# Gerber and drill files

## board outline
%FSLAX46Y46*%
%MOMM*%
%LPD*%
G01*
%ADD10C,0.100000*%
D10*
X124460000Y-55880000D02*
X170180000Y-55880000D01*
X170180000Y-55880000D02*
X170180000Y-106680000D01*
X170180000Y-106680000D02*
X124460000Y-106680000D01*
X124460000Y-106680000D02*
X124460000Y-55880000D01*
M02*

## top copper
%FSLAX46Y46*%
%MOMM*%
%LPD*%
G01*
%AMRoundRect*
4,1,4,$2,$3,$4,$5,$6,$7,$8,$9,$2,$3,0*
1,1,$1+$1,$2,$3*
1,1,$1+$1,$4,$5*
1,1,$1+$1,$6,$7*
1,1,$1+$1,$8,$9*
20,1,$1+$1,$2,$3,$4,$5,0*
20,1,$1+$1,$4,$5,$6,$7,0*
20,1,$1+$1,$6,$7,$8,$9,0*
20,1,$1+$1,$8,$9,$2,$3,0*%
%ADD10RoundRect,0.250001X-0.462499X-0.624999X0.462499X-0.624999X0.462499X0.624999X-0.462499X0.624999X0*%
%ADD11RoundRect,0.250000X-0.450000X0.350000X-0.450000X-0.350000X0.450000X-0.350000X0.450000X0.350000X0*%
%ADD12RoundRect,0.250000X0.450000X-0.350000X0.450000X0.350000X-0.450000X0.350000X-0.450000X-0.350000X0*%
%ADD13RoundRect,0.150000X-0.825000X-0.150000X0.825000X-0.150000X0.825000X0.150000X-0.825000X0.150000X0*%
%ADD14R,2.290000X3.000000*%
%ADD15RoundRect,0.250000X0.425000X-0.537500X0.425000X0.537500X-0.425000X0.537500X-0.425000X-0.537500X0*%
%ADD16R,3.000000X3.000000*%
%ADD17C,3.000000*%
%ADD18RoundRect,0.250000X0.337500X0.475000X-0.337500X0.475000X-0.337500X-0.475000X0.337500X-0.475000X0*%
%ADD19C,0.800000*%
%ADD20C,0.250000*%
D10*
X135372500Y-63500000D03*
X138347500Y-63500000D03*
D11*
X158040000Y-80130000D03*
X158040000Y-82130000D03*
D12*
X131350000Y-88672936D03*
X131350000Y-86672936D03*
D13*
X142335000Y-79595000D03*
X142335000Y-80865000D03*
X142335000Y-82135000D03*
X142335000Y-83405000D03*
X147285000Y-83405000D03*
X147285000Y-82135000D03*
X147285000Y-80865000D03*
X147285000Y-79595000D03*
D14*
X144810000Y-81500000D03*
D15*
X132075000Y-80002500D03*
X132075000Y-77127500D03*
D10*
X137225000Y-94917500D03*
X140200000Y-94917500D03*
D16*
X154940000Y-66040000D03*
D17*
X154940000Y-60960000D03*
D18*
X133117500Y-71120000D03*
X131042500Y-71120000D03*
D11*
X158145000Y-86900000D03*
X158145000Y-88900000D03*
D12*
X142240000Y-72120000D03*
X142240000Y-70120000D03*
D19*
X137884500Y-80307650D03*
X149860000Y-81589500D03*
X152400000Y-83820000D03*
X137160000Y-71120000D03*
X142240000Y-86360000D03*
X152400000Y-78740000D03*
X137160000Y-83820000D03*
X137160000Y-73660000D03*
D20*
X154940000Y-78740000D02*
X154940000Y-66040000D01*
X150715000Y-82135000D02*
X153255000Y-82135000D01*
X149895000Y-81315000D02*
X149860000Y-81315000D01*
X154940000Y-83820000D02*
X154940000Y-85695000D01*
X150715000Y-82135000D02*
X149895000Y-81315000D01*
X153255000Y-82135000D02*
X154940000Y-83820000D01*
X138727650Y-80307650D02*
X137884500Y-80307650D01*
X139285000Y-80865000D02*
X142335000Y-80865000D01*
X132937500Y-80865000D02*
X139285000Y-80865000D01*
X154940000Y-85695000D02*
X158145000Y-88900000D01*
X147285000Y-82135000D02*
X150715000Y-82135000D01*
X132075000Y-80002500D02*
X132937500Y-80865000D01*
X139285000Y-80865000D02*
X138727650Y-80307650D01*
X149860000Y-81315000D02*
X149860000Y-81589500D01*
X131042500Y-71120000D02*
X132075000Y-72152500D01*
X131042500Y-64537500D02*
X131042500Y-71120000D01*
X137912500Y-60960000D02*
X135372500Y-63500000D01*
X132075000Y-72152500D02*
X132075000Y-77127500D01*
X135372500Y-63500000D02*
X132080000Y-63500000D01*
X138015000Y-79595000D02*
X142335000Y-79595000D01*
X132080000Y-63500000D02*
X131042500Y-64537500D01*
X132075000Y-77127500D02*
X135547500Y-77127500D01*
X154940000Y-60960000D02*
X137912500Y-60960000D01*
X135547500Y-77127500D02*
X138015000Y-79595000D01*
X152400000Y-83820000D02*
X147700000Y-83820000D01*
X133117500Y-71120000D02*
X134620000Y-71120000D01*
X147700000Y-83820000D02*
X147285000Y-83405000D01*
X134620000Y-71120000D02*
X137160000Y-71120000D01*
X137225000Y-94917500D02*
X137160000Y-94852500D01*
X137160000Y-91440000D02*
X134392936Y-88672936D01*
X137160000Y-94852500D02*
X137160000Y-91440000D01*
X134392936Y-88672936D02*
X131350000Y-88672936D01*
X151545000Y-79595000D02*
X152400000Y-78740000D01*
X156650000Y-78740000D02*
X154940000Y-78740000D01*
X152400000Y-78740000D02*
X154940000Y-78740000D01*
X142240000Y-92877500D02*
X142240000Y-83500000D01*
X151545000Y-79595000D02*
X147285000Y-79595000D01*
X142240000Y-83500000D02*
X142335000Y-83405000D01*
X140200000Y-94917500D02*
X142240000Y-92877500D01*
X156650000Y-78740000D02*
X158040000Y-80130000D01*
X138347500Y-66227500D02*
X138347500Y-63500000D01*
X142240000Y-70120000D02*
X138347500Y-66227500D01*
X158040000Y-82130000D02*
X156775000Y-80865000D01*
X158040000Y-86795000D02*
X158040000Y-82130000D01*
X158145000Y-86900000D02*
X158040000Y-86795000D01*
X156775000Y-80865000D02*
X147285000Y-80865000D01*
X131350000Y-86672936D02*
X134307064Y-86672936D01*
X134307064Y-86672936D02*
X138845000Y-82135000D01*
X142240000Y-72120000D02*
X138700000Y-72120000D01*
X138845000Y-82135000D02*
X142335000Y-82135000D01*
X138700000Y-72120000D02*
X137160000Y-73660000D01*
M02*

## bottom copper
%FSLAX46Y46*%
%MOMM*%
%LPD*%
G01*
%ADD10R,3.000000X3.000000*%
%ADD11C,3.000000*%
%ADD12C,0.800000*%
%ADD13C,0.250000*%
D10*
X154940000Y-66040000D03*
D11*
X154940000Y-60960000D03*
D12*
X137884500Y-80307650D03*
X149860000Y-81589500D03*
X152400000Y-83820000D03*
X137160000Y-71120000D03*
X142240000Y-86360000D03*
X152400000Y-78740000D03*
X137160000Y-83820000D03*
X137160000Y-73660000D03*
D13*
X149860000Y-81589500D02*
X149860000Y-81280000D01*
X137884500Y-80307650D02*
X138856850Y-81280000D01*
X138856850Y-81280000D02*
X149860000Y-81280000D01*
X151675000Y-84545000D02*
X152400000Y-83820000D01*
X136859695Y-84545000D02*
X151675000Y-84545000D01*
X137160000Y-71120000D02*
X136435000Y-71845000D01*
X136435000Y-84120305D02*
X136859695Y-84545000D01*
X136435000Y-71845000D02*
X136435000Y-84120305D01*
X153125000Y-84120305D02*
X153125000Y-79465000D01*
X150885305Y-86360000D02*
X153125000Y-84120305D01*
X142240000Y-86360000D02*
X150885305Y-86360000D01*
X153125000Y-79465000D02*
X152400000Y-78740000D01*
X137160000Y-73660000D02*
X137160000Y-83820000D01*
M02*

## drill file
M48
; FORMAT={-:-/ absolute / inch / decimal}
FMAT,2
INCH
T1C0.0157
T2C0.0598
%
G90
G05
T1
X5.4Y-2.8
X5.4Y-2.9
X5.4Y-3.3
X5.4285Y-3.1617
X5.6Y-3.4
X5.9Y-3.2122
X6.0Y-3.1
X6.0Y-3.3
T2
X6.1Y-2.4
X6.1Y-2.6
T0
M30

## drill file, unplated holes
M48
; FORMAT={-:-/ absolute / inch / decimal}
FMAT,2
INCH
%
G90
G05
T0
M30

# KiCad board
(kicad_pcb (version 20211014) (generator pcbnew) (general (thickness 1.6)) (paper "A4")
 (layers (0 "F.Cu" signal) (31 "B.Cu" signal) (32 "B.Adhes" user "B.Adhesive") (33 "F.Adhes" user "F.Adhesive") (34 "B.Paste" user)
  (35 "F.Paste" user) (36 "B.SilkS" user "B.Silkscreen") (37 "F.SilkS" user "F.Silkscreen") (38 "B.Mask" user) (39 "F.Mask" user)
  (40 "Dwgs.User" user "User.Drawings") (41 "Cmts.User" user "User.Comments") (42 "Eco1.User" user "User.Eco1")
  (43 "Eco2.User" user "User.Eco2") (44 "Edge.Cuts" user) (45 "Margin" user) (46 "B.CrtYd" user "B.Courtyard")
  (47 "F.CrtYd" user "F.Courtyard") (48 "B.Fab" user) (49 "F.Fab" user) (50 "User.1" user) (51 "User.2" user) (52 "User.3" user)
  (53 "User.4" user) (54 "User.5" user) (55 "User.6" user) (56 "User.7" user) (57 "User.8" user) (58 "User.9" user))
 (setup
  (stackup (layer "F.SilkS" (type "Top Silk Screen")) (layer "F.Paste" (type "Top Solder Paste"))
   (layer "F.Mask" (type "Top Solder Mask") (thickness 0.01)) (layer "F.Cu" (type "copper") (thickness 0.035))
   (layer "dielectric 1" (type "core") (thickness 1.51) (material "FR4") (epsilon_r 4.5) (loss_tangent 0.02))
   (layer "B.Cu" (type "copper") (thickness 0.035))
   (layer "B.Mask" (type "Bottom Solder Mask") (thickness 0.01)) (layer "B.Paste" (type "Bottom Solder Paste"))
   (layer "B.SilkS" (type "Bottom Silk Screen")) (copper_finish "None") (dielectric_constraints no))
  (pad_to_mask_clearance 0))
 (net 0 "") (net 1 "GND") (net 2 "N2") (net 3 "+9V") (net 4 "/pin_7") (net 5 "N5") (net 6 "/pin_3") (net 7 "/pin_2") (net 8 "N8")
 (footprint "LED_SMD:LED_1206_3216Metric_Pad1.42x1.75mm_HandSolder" (layer "F.Cu") (at 136.86 63.5)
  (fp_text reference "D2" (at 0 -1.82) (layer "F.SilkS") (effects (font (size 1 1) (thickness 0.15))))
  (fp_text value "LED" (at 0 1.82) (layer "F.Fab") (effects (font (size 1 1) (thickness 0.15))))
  (pad "1" smd roundrect (at -1.4875 0) (size 1.425 1.75) (layers "F.Cu" "F.Paste" "F.Mask") (roundrect_rratio 0.175439) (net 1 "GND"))
  (pad "2" smd roundrect (at 1.4875 0) (size 1.425 1.75) (layers "F.Cu" "F.Paste" "F.Mask") (roundrect_rratio 0.175439) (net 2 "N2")))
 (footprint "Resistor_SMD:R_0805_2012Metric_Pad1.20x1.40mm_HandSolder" (layer "F.Cu") (at 158.04 81.13 -90)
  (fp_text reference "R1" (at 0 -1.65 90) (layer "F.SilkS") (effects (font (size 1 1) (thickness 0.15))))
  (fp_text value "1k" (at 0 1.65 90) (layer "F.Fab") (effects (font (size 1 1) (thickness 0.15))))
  (pad "1" smd roundrect (at -1 0 270) (size 1.2 1.4) (layers "F.Cu" "F.Paste" "F.Mask") (roundrect_rratio 0.208333) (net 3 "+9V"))
  (pad "2" smd roundrect (at 1 0 270) (size 1.2 1.4) (layers "F.Cu" "F.Paste" "F.Mask") (roundrect_rratio 0.208333) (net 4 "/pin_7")))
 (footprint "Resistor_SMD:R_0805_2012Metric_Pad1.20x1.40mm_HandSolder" (layer "F.Cu") (at 131.35 87.672936 90)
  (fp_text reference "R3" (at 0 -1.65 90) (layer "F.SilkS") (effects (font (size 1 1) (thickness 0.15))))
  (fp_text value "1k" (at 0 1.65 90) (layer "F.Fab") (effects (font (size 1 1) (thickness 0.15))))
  (pad "1" smd roundrect (at -1 0 90) (size 1.2 1.4) (layers "F.Cu" "F.Paste" "F.Mask") (roundrect_rratio 0.208333) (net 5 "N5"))
  (pad "2" smd roundrect (at 1 0 90) (size 1.2 1.4) (layers "F.Cu" "F.Paste" "F.Mask") (roundrect_rratio 0.208333) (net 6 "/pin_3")))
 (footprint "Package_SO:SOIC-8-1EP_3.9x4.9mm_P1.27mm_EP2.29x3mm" (layer "F.Cu") (at 144.81 81.5)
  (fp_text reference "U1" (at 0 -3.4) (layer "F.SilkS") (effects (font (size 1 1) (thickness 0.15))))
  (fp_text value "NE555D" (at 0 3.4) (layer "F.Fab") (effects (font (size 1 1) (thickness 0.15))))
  (pad "" smd roundrect (at -0.57 -0.75) (size 0.92 1.21) (layers "F.Paste") (roundrect_rratio 0.25))
  (pad "" smd roundrect (at 0.57 0.75) (size 0.92 1.21) (layers "F.Paste") (roundrect_rratio 0.25))
  (pad "" smd roundrect (at -0.57 0.75) (size 0.92 1.21) (layers "F.Paste") (roundrect_rratio 0.25))
  (pad "" smd roundrect (at 0.57 -0.75) (size 0.92 1.21) (layers "F.Paste") (roundrect_rratio 0.25))
  (pad "1" smd roundrect (at -2.475 -1.905) (size 1.95 0.6) (layers "F.Cu" "F.Paste" "F.Mask") (roundrect_rratio 0.25) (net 1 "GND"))
  (pad "2" smd roundrect (at -2.475 -0.635) (size 1.95 0.6) (layers "F.Cu" "F.Paste" "F.Mask") (roundrect_rratio 0.25) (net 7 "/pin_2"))
  (pad "3" smd roundrect (at -2.475 0.635) (size 1.95 0.6) (layers "F.Cu" "F.Paste" "F.Mask") (roundrect_rratio 0.25) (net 6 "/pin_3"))
  (pad "4" smd roundrect (at -2.475 1.905) (size 1.95 0.6) (layers "F.Cu" "F.Paste" "F.Mask") (roundrect_rratio 0.25) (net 3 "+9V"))
  (pad "5" smd roundrect (at 2.475 1.905) (size 1.95 0.6) (layers "F.Cu" "F.Paste" "F.Mask") (roundrect_rratio 0.25) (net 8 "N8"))
  (pad "6" smd roundrect (at 2.475 0.635) (size 1.95 0.6) (layers "F.Cu" "F.Paste" "F.Mask") (roundrect_rratio 0.25) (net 7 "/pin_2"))
  (pad "7" smd roundrect (at 2.475 -0.635) (size 1.95 0.6) (layers "F.Cu" "F.Paste" "F.Mask") (roundrect_rratio 0.25) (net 4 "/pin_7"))
  (pad "8" smd roundrect (at 2.475 -1.905) (size 1.95 0.6) (layers "F.Cu" "F.Paste" "F.Mask") (roundrect_rratio 0.25) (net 3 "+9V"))
  (pad "9" smd rect (at 0 0) (size 2.29 3) (layers "F.Cu" "F.Mask")))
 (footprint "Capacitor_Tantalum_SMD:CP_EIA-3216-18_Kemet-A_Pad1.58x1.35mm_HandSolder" (layer "F.Cu") (at 132.075 78.565 90)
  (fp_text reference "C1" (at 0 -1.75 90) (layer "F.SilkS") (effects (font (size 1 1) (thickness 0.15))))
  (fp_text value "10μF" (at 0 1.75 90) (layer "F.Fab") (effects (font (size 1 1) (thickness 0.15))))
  (pad "1" smd roundrect (at -1.4375 0 90) (size 1.575 1.35) (layers "F.Cu" "F.Paste" "F.Mask") (roundrect_rratio 0.185185) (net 7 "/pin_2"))
  (pad "2" smd roundrect (at 1.4375 0 90) (size 1.575 1.35) (layers "F.Cu" "F.Paste" "F.Mask") (roundrect_rratio 0.185185) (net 1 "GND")))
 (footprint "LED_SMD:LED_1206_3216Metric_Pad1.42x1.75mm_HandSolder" (layer "F.Cu") (at 138.7125 94.9175)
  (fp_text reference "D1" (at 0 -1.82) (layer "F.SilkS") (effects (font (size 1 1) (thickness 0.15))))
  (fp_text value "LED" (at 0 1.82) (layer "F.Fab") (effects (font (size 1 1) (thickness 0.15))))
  (pad "1" smd roundrect (at -1.4875 0) (size 1.425 1.75) (layers "F.Cu" "F.Paste" "F.Mask") (roundrect_rratio 0.175439) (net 5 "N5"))
  (pad "2" smd roundrect (at 1.4875 0) (size 1.425 1.75) (layers "F.Cu" "F.Paste" "F.Mask") (roundrect_rratio 0.175439) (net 3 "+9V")))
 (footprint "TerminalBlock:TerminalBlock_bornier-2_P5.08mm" (layer "F.Cu") (at 154.94 66.04 90)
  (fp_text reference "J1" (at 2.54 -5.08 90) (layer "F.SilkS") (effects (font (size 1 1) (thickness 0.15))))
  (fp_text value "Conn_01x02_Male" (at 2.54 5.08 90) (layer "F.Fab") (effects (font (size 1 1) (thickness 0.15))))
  (pad "1" thru_hole rect (at 0 0 90) (size 3 3) (drill 1.52) (layers *.Cu *.Mask) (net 3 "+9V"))
  (pad "2" thru_hole circle (at 5.08 0 90) (size 3 3) (drill 1.52) (layers *.Cu *.Mask) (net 1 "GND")))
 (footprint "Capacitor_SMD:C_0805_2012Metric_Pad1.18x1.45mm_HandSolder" (layer "F.Cu") (at 132.08 71.12 180)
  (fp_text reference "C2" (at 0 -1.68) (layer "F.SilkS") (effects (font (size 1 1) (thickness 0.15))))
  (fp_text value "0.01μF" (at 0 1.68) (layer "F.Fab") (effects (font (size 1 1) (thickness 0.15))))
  (pad "1" smd roundrect (at -1.0375 0 180) (size 1.175 1.45) (layers "F.Cu" "F.Paste" "F.Mask") (roundrect_rratio 0.212766) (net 8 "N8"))
  (pad "2" smd roundrect (at 1.0375 0 180) (size 1.175 1.45) (layers "F.Cu" "F.Paste" "F.Mask") (roundrect_rratio 0.212766) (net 1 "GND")))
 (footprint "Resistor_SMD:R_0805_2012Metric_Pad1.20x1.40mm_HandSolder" (layer "F.Cu") (at 158.145 87.9 -90)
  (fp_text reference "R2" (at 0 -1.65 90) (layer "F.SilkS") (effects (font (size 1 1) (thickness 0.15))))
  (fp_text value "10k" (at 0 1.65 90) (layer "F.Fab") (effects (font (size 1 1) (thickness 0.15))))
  (pad "1" smd roundrect (at -1 0 270) (size 1.2 1.4) (layers "F.Cu" "F.Paste" "F.Mask") (roundrect_rratio 0.208333) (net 4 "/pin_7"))
  (pad "2" smd roundrect (at 1 0 270) (size 1.2 1.4) (layers "F.Cu" "F.Paste" "F.Mask") (roundrect_rratio 0.208333) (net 7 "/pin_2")))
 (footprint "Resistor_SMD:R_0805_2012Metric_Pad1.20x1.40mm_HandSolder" (layer "F.Cu") (at 142.24 71.12 90)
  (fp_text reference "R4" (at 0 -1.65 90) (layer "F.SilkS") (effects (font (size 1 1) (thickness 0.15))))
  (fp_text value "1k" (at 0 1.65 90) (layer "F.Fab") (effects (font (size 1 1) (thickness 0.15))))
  (pad "1" smd roundrect (at -1 0 90) (size 1.2 1.4) (layers "F.Cu" "F.Paste" "F.Mask") (roundrect_rratio 0.208333) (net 6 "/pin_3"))
  (pad "2" smd roundrect (at 1 0 90) (size 1.2 1.4) (layers "F.Cu" "F.Paste" "F.Mask") (roundrect_rratio 0.208333) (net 2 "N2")))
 (gr_rect (start 124.46 55.88) (end 170.18 106.68) (layer "Edge.Cuts") (width 0.1) (fill none))
 (segment (start 150.715 82.135) (end 153.255 82.135) (width 0.25) (layer "F.Cu") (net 7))
 (segment (start 149.895 81.315) (end 149.86 81.315) (width 0.25) (layer "F.Cu") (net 7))
 (segment (start 154.94 83.82) (end 154.94 85.695) (width 0.25) (layer "F.Cu") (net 7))
 (segment (start 150.715 82.135) (end 149.895 81.315) (width 0.25) (layer "F.Cu") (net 7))
 (segment (start 153.255 82.135) (end 154.94 83.82) (width 0.25) (layer "F.Cu") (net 7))
 (segment (start 138.72765 80.30765) (end 137.8845 80.30765) (width 0.25) (layer "F.Cu") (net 7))
 (segment (start 139.285 80.865) (end 142.335 80.865) (width 0.25) (layer "F.Cu") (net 7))
 (segment (start 132.9375 80.865) (end 139.285 80.865) (width 0.25) (layer "F.Cu") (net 7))
 (segment (start 154.94 85.695) (end 158.145 88.9) (width 0.25) (layer "F.Cu") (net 7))
 (segment (start 147.285 82.135) (end 150.715 82.135) (width 0.25) (layer "F.Cu") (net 7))
 (segment (start 132.075 80.0025) (end 132.9375 80.865) (width 0.25) (layer "F.Cu") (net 7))
 (segment (start 139.285 80.865) (end 138.72765 80.30765) (width 0.25) (layer "F.Cu") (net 7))
 (segment (start 149.86 81.315) (end 149.86 81.5895) (width 0.25) (layer "F.Cu") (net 7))
 (via (at 137.8845 80.30765) (size 0.8) (drill 0.4) (layers "F.Cu" "B.Cu") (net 7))
 (via (at 149.86 81.5895) (size 0.8) (drill 0.4) (layers "F.Cu" "B.Cu") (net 7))
 (segment (start 149.86 81.5895) (end 149.86 81.28) (width 0.25) (layer "B.Cu") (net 7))
 (segment (start 137.8845 80.30765) (end 138.85685 81.28) (width 0.25) (layer "B.Cu") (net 7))
 (segment (start 138.85685 81.28) (end 149.86 81.28) (width 0.25) (layer "B.Cu") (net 7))
 (segment (start 131.0425 71.12) (end 132.075 72.1525) (width 0.25) (layer "F.Cu") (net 1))
 (segment (start 131.0425 64.5375) (end 131.0425 71.12) (width 0.25) (layer "F.Cu") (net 1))
 (segment (start 137.9125 60.96) (end 135.3725 63.5) (width 0.25) (layer "F.Cu") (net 1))
 (segment (start 132.075 72.1525) (end 132.075 77.1275) (width 0.25) (layer "F.Cu") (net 1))
 (segment (start 135.3725 63.5) (end 132.08 63.5) (width 0.25) (layer "F.Cu") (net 1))
 (segment (start 138.015 79.595) (end 142.335 79.595) (width 0.25) (layer "F.Cu") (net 1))
 (segment (start 132.08 63.5) (end 131.0425 64.5375) (width 0.25) (layer "F.Cu") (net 1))
 (segment (start 132.075 77.1275) (end 135.5475 77.1275) (width 0.25) (layer "F.Cu") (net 1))
 (segment (start 154.94 60.96) (end 137.9125 60.96) (width 0.25) (layer "F.Cu") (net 1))
 (segment (start 135.5475 77.1275) (end 138.015 79.595) (width 0.25) (layer "F.Cu") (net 1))
 (segment (start 152.4 83.82) (end 147.7 83.82) (width 0.25) (layer "F.Cu") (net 8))
 (segment (start 133.1175 71.12) (end 134.62 71.12) (width 0.25) (layer "F.Cu") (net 8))
 (segment (start 147.7 83.82) (end 147.285 83.405) (width 0.25) (layer "F.Cu") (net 8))
 (segment (start 134.62 71.12) (end 137.16 71.12) (width 0.25) (layer "F.Cu") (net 8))
 (via (at 152.4 83.82) (size 0.8) (drill 0.4) (layers "F.Cu" "B.Cu") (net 8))
 (via (at 137.16 71.12) (size 0.8) (drill 0.4) (layers "F.Cu" "B.Cu") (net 8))
 (segment (start 151.675 84.545) (end 152.4 83.82) (width 0.25) (layer "B.Cu") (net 8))
 (segment (start 136.859695 84.545) (end 151.675 84.545) (width 0.25) (layer "B.Cu") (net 8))
 (segment (start 137.16 71.12) (end 136.435 71.845) (width 0.25) (layer "B.Cu") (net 8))
 (segment (start 136.435 84.120305) (end 136.859695 84.545) (width 0.25) (layer "B.Cu") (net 8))
 (segment (start 136.435 71.845) (end 136.435 84.120305) (width 0.25) (layer "B.Cu") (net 8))
 (segment (start 137.225 94.9175) (end 137.16 94.8525) (width 0.25) (layer "F.Cu") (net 5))
 (segment (start 137.16 91.44) (end 134.392936 88.672936) (width 0.25) (layer "F.Cu") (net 5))
 (segment (start 137.16 94.8525) (end 137.16 91.44) (width 0.25) (layer "F.Cu") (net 5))
 (segment (start 134.392936 88.672936) (end 131.35 88.672936) (width 0.25) (layer "F.Cu") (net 5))
 (segment (start 151.545 79.595) (end 152.4 78.74) (width 0.25) (layer "F.Cu") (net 3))
 (segment (start 156.65 78.74) (end 154.94 78.74) (width 0.25) (layer "F.Cu") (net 3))
 (segment (start 154.94 78.74) (end 154.94 66.04) (width 0.25) (layer "F.Cu") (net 3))
 (segment (start 152.4 78.74) (end 154.94 78.74) (width 0.25) (layer "F.Cu") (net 3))
 (segment (start 142.24 92.8775) (end 142.24 83.5) (width 0.25) (layer "F.Cu") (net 3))
 (segment (start 151.545 79.595) (end 147.285 79.595) (width 0.25) (layer "F.Cu") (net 3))
 (segment (start 142.24 83.5) (end 142.335 83.405) (width 0.25) (layer "F.Cu") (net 3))
 (segment (start 140.2 94.9175) (end 142.24 92.8775) (width 0.25) (layer "F.Cu") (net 3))
 (segment (start 156.65 78.74) (end 158.04 80.13) (width 0.25) (layer "F.Cu") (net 3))
 (via (at 142.24 86.36) (size 0.8) (drill 0.4) (layers "F.Cu" "B.Cu") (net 3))
 (via (at 152.4 78.74) (size 0.8) (drill 0.4) (layers "F.Cu" "B.Cu") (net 3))
 (segment (start 153.125 84.120305) (end 153.125 79.465) (width 0.25) (layer "B.Cu") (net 3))
 (segment (start 150.885305 86.36) (end 153.125 84.120305) (width 0.25) (layer "B.Cu") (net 3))
 (segment (start 142.24 86.36) (end 150.885305 86.36) (width 0.25) (layer "B.Cu") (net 3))
 (segment (start 153.125 79.465) (end 152.4 78.74) (width 0.25) (layer "B.Cu") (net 3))
 (segment (start 138.3475 66.2275) (end 138.3475 63.5) (width 0.25) (layer "F.Cu") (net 2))
 (segment (start 142.24 70.12) (end 138.3475 66.2275) (width 0.25) (layer "F.Cu") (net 2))
 (segment (start 158.04 82.13) (end 156.775 80.865) (width 0.25) (layer "F.Cu") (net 4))
 (segment (start 158.04 86.795) (end 158.04 82.13) (width 0.25) (layer "F.Cu") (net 4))
 (segment (start 158.145 86.9) (end 158.04 86.795) (width 0.25) (layer "F.Cu") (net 4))
 (segment (start 156.775 80.865) (end 147.285 80.865) (width 0.25) (layer "F.Cu") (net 4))
 (segment (start 131.35 86.672936) (end 134.307064 86.672936) (width 0.25) (layer "F.Cu") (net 6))
 (segment (start 134.307064 86.672936) (end 138.845 82.135) (width 0.25) (layer "F.Cu") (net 6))
 (segment (start 142.24 72.12) (end 138.7 72.12) (width 0.25) (layer "F.Cu") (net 6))
 (segment (start 138.845 82.135) (end 142.335 82.135) (width 0.25) (layer "F.Cu") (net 6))
 (segment (start 138.7 72.12) (end 137.16 73.66) (width 0.25) (layer "F.Cu") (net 6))
 (via (at 137.16 83.82) (size 0.8) (drill 0.4) (layers "F.Cu" "B.Cu") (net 6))
 (via (at 137.16 73.66) (size 0.8) (drill 0.4) (layers "F.Cu" "B.Cu") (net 6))
 (segment (start 137.16 73.66) (end 137.16 83.82) (width 0.25) (layer "B.Cu") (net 6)))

